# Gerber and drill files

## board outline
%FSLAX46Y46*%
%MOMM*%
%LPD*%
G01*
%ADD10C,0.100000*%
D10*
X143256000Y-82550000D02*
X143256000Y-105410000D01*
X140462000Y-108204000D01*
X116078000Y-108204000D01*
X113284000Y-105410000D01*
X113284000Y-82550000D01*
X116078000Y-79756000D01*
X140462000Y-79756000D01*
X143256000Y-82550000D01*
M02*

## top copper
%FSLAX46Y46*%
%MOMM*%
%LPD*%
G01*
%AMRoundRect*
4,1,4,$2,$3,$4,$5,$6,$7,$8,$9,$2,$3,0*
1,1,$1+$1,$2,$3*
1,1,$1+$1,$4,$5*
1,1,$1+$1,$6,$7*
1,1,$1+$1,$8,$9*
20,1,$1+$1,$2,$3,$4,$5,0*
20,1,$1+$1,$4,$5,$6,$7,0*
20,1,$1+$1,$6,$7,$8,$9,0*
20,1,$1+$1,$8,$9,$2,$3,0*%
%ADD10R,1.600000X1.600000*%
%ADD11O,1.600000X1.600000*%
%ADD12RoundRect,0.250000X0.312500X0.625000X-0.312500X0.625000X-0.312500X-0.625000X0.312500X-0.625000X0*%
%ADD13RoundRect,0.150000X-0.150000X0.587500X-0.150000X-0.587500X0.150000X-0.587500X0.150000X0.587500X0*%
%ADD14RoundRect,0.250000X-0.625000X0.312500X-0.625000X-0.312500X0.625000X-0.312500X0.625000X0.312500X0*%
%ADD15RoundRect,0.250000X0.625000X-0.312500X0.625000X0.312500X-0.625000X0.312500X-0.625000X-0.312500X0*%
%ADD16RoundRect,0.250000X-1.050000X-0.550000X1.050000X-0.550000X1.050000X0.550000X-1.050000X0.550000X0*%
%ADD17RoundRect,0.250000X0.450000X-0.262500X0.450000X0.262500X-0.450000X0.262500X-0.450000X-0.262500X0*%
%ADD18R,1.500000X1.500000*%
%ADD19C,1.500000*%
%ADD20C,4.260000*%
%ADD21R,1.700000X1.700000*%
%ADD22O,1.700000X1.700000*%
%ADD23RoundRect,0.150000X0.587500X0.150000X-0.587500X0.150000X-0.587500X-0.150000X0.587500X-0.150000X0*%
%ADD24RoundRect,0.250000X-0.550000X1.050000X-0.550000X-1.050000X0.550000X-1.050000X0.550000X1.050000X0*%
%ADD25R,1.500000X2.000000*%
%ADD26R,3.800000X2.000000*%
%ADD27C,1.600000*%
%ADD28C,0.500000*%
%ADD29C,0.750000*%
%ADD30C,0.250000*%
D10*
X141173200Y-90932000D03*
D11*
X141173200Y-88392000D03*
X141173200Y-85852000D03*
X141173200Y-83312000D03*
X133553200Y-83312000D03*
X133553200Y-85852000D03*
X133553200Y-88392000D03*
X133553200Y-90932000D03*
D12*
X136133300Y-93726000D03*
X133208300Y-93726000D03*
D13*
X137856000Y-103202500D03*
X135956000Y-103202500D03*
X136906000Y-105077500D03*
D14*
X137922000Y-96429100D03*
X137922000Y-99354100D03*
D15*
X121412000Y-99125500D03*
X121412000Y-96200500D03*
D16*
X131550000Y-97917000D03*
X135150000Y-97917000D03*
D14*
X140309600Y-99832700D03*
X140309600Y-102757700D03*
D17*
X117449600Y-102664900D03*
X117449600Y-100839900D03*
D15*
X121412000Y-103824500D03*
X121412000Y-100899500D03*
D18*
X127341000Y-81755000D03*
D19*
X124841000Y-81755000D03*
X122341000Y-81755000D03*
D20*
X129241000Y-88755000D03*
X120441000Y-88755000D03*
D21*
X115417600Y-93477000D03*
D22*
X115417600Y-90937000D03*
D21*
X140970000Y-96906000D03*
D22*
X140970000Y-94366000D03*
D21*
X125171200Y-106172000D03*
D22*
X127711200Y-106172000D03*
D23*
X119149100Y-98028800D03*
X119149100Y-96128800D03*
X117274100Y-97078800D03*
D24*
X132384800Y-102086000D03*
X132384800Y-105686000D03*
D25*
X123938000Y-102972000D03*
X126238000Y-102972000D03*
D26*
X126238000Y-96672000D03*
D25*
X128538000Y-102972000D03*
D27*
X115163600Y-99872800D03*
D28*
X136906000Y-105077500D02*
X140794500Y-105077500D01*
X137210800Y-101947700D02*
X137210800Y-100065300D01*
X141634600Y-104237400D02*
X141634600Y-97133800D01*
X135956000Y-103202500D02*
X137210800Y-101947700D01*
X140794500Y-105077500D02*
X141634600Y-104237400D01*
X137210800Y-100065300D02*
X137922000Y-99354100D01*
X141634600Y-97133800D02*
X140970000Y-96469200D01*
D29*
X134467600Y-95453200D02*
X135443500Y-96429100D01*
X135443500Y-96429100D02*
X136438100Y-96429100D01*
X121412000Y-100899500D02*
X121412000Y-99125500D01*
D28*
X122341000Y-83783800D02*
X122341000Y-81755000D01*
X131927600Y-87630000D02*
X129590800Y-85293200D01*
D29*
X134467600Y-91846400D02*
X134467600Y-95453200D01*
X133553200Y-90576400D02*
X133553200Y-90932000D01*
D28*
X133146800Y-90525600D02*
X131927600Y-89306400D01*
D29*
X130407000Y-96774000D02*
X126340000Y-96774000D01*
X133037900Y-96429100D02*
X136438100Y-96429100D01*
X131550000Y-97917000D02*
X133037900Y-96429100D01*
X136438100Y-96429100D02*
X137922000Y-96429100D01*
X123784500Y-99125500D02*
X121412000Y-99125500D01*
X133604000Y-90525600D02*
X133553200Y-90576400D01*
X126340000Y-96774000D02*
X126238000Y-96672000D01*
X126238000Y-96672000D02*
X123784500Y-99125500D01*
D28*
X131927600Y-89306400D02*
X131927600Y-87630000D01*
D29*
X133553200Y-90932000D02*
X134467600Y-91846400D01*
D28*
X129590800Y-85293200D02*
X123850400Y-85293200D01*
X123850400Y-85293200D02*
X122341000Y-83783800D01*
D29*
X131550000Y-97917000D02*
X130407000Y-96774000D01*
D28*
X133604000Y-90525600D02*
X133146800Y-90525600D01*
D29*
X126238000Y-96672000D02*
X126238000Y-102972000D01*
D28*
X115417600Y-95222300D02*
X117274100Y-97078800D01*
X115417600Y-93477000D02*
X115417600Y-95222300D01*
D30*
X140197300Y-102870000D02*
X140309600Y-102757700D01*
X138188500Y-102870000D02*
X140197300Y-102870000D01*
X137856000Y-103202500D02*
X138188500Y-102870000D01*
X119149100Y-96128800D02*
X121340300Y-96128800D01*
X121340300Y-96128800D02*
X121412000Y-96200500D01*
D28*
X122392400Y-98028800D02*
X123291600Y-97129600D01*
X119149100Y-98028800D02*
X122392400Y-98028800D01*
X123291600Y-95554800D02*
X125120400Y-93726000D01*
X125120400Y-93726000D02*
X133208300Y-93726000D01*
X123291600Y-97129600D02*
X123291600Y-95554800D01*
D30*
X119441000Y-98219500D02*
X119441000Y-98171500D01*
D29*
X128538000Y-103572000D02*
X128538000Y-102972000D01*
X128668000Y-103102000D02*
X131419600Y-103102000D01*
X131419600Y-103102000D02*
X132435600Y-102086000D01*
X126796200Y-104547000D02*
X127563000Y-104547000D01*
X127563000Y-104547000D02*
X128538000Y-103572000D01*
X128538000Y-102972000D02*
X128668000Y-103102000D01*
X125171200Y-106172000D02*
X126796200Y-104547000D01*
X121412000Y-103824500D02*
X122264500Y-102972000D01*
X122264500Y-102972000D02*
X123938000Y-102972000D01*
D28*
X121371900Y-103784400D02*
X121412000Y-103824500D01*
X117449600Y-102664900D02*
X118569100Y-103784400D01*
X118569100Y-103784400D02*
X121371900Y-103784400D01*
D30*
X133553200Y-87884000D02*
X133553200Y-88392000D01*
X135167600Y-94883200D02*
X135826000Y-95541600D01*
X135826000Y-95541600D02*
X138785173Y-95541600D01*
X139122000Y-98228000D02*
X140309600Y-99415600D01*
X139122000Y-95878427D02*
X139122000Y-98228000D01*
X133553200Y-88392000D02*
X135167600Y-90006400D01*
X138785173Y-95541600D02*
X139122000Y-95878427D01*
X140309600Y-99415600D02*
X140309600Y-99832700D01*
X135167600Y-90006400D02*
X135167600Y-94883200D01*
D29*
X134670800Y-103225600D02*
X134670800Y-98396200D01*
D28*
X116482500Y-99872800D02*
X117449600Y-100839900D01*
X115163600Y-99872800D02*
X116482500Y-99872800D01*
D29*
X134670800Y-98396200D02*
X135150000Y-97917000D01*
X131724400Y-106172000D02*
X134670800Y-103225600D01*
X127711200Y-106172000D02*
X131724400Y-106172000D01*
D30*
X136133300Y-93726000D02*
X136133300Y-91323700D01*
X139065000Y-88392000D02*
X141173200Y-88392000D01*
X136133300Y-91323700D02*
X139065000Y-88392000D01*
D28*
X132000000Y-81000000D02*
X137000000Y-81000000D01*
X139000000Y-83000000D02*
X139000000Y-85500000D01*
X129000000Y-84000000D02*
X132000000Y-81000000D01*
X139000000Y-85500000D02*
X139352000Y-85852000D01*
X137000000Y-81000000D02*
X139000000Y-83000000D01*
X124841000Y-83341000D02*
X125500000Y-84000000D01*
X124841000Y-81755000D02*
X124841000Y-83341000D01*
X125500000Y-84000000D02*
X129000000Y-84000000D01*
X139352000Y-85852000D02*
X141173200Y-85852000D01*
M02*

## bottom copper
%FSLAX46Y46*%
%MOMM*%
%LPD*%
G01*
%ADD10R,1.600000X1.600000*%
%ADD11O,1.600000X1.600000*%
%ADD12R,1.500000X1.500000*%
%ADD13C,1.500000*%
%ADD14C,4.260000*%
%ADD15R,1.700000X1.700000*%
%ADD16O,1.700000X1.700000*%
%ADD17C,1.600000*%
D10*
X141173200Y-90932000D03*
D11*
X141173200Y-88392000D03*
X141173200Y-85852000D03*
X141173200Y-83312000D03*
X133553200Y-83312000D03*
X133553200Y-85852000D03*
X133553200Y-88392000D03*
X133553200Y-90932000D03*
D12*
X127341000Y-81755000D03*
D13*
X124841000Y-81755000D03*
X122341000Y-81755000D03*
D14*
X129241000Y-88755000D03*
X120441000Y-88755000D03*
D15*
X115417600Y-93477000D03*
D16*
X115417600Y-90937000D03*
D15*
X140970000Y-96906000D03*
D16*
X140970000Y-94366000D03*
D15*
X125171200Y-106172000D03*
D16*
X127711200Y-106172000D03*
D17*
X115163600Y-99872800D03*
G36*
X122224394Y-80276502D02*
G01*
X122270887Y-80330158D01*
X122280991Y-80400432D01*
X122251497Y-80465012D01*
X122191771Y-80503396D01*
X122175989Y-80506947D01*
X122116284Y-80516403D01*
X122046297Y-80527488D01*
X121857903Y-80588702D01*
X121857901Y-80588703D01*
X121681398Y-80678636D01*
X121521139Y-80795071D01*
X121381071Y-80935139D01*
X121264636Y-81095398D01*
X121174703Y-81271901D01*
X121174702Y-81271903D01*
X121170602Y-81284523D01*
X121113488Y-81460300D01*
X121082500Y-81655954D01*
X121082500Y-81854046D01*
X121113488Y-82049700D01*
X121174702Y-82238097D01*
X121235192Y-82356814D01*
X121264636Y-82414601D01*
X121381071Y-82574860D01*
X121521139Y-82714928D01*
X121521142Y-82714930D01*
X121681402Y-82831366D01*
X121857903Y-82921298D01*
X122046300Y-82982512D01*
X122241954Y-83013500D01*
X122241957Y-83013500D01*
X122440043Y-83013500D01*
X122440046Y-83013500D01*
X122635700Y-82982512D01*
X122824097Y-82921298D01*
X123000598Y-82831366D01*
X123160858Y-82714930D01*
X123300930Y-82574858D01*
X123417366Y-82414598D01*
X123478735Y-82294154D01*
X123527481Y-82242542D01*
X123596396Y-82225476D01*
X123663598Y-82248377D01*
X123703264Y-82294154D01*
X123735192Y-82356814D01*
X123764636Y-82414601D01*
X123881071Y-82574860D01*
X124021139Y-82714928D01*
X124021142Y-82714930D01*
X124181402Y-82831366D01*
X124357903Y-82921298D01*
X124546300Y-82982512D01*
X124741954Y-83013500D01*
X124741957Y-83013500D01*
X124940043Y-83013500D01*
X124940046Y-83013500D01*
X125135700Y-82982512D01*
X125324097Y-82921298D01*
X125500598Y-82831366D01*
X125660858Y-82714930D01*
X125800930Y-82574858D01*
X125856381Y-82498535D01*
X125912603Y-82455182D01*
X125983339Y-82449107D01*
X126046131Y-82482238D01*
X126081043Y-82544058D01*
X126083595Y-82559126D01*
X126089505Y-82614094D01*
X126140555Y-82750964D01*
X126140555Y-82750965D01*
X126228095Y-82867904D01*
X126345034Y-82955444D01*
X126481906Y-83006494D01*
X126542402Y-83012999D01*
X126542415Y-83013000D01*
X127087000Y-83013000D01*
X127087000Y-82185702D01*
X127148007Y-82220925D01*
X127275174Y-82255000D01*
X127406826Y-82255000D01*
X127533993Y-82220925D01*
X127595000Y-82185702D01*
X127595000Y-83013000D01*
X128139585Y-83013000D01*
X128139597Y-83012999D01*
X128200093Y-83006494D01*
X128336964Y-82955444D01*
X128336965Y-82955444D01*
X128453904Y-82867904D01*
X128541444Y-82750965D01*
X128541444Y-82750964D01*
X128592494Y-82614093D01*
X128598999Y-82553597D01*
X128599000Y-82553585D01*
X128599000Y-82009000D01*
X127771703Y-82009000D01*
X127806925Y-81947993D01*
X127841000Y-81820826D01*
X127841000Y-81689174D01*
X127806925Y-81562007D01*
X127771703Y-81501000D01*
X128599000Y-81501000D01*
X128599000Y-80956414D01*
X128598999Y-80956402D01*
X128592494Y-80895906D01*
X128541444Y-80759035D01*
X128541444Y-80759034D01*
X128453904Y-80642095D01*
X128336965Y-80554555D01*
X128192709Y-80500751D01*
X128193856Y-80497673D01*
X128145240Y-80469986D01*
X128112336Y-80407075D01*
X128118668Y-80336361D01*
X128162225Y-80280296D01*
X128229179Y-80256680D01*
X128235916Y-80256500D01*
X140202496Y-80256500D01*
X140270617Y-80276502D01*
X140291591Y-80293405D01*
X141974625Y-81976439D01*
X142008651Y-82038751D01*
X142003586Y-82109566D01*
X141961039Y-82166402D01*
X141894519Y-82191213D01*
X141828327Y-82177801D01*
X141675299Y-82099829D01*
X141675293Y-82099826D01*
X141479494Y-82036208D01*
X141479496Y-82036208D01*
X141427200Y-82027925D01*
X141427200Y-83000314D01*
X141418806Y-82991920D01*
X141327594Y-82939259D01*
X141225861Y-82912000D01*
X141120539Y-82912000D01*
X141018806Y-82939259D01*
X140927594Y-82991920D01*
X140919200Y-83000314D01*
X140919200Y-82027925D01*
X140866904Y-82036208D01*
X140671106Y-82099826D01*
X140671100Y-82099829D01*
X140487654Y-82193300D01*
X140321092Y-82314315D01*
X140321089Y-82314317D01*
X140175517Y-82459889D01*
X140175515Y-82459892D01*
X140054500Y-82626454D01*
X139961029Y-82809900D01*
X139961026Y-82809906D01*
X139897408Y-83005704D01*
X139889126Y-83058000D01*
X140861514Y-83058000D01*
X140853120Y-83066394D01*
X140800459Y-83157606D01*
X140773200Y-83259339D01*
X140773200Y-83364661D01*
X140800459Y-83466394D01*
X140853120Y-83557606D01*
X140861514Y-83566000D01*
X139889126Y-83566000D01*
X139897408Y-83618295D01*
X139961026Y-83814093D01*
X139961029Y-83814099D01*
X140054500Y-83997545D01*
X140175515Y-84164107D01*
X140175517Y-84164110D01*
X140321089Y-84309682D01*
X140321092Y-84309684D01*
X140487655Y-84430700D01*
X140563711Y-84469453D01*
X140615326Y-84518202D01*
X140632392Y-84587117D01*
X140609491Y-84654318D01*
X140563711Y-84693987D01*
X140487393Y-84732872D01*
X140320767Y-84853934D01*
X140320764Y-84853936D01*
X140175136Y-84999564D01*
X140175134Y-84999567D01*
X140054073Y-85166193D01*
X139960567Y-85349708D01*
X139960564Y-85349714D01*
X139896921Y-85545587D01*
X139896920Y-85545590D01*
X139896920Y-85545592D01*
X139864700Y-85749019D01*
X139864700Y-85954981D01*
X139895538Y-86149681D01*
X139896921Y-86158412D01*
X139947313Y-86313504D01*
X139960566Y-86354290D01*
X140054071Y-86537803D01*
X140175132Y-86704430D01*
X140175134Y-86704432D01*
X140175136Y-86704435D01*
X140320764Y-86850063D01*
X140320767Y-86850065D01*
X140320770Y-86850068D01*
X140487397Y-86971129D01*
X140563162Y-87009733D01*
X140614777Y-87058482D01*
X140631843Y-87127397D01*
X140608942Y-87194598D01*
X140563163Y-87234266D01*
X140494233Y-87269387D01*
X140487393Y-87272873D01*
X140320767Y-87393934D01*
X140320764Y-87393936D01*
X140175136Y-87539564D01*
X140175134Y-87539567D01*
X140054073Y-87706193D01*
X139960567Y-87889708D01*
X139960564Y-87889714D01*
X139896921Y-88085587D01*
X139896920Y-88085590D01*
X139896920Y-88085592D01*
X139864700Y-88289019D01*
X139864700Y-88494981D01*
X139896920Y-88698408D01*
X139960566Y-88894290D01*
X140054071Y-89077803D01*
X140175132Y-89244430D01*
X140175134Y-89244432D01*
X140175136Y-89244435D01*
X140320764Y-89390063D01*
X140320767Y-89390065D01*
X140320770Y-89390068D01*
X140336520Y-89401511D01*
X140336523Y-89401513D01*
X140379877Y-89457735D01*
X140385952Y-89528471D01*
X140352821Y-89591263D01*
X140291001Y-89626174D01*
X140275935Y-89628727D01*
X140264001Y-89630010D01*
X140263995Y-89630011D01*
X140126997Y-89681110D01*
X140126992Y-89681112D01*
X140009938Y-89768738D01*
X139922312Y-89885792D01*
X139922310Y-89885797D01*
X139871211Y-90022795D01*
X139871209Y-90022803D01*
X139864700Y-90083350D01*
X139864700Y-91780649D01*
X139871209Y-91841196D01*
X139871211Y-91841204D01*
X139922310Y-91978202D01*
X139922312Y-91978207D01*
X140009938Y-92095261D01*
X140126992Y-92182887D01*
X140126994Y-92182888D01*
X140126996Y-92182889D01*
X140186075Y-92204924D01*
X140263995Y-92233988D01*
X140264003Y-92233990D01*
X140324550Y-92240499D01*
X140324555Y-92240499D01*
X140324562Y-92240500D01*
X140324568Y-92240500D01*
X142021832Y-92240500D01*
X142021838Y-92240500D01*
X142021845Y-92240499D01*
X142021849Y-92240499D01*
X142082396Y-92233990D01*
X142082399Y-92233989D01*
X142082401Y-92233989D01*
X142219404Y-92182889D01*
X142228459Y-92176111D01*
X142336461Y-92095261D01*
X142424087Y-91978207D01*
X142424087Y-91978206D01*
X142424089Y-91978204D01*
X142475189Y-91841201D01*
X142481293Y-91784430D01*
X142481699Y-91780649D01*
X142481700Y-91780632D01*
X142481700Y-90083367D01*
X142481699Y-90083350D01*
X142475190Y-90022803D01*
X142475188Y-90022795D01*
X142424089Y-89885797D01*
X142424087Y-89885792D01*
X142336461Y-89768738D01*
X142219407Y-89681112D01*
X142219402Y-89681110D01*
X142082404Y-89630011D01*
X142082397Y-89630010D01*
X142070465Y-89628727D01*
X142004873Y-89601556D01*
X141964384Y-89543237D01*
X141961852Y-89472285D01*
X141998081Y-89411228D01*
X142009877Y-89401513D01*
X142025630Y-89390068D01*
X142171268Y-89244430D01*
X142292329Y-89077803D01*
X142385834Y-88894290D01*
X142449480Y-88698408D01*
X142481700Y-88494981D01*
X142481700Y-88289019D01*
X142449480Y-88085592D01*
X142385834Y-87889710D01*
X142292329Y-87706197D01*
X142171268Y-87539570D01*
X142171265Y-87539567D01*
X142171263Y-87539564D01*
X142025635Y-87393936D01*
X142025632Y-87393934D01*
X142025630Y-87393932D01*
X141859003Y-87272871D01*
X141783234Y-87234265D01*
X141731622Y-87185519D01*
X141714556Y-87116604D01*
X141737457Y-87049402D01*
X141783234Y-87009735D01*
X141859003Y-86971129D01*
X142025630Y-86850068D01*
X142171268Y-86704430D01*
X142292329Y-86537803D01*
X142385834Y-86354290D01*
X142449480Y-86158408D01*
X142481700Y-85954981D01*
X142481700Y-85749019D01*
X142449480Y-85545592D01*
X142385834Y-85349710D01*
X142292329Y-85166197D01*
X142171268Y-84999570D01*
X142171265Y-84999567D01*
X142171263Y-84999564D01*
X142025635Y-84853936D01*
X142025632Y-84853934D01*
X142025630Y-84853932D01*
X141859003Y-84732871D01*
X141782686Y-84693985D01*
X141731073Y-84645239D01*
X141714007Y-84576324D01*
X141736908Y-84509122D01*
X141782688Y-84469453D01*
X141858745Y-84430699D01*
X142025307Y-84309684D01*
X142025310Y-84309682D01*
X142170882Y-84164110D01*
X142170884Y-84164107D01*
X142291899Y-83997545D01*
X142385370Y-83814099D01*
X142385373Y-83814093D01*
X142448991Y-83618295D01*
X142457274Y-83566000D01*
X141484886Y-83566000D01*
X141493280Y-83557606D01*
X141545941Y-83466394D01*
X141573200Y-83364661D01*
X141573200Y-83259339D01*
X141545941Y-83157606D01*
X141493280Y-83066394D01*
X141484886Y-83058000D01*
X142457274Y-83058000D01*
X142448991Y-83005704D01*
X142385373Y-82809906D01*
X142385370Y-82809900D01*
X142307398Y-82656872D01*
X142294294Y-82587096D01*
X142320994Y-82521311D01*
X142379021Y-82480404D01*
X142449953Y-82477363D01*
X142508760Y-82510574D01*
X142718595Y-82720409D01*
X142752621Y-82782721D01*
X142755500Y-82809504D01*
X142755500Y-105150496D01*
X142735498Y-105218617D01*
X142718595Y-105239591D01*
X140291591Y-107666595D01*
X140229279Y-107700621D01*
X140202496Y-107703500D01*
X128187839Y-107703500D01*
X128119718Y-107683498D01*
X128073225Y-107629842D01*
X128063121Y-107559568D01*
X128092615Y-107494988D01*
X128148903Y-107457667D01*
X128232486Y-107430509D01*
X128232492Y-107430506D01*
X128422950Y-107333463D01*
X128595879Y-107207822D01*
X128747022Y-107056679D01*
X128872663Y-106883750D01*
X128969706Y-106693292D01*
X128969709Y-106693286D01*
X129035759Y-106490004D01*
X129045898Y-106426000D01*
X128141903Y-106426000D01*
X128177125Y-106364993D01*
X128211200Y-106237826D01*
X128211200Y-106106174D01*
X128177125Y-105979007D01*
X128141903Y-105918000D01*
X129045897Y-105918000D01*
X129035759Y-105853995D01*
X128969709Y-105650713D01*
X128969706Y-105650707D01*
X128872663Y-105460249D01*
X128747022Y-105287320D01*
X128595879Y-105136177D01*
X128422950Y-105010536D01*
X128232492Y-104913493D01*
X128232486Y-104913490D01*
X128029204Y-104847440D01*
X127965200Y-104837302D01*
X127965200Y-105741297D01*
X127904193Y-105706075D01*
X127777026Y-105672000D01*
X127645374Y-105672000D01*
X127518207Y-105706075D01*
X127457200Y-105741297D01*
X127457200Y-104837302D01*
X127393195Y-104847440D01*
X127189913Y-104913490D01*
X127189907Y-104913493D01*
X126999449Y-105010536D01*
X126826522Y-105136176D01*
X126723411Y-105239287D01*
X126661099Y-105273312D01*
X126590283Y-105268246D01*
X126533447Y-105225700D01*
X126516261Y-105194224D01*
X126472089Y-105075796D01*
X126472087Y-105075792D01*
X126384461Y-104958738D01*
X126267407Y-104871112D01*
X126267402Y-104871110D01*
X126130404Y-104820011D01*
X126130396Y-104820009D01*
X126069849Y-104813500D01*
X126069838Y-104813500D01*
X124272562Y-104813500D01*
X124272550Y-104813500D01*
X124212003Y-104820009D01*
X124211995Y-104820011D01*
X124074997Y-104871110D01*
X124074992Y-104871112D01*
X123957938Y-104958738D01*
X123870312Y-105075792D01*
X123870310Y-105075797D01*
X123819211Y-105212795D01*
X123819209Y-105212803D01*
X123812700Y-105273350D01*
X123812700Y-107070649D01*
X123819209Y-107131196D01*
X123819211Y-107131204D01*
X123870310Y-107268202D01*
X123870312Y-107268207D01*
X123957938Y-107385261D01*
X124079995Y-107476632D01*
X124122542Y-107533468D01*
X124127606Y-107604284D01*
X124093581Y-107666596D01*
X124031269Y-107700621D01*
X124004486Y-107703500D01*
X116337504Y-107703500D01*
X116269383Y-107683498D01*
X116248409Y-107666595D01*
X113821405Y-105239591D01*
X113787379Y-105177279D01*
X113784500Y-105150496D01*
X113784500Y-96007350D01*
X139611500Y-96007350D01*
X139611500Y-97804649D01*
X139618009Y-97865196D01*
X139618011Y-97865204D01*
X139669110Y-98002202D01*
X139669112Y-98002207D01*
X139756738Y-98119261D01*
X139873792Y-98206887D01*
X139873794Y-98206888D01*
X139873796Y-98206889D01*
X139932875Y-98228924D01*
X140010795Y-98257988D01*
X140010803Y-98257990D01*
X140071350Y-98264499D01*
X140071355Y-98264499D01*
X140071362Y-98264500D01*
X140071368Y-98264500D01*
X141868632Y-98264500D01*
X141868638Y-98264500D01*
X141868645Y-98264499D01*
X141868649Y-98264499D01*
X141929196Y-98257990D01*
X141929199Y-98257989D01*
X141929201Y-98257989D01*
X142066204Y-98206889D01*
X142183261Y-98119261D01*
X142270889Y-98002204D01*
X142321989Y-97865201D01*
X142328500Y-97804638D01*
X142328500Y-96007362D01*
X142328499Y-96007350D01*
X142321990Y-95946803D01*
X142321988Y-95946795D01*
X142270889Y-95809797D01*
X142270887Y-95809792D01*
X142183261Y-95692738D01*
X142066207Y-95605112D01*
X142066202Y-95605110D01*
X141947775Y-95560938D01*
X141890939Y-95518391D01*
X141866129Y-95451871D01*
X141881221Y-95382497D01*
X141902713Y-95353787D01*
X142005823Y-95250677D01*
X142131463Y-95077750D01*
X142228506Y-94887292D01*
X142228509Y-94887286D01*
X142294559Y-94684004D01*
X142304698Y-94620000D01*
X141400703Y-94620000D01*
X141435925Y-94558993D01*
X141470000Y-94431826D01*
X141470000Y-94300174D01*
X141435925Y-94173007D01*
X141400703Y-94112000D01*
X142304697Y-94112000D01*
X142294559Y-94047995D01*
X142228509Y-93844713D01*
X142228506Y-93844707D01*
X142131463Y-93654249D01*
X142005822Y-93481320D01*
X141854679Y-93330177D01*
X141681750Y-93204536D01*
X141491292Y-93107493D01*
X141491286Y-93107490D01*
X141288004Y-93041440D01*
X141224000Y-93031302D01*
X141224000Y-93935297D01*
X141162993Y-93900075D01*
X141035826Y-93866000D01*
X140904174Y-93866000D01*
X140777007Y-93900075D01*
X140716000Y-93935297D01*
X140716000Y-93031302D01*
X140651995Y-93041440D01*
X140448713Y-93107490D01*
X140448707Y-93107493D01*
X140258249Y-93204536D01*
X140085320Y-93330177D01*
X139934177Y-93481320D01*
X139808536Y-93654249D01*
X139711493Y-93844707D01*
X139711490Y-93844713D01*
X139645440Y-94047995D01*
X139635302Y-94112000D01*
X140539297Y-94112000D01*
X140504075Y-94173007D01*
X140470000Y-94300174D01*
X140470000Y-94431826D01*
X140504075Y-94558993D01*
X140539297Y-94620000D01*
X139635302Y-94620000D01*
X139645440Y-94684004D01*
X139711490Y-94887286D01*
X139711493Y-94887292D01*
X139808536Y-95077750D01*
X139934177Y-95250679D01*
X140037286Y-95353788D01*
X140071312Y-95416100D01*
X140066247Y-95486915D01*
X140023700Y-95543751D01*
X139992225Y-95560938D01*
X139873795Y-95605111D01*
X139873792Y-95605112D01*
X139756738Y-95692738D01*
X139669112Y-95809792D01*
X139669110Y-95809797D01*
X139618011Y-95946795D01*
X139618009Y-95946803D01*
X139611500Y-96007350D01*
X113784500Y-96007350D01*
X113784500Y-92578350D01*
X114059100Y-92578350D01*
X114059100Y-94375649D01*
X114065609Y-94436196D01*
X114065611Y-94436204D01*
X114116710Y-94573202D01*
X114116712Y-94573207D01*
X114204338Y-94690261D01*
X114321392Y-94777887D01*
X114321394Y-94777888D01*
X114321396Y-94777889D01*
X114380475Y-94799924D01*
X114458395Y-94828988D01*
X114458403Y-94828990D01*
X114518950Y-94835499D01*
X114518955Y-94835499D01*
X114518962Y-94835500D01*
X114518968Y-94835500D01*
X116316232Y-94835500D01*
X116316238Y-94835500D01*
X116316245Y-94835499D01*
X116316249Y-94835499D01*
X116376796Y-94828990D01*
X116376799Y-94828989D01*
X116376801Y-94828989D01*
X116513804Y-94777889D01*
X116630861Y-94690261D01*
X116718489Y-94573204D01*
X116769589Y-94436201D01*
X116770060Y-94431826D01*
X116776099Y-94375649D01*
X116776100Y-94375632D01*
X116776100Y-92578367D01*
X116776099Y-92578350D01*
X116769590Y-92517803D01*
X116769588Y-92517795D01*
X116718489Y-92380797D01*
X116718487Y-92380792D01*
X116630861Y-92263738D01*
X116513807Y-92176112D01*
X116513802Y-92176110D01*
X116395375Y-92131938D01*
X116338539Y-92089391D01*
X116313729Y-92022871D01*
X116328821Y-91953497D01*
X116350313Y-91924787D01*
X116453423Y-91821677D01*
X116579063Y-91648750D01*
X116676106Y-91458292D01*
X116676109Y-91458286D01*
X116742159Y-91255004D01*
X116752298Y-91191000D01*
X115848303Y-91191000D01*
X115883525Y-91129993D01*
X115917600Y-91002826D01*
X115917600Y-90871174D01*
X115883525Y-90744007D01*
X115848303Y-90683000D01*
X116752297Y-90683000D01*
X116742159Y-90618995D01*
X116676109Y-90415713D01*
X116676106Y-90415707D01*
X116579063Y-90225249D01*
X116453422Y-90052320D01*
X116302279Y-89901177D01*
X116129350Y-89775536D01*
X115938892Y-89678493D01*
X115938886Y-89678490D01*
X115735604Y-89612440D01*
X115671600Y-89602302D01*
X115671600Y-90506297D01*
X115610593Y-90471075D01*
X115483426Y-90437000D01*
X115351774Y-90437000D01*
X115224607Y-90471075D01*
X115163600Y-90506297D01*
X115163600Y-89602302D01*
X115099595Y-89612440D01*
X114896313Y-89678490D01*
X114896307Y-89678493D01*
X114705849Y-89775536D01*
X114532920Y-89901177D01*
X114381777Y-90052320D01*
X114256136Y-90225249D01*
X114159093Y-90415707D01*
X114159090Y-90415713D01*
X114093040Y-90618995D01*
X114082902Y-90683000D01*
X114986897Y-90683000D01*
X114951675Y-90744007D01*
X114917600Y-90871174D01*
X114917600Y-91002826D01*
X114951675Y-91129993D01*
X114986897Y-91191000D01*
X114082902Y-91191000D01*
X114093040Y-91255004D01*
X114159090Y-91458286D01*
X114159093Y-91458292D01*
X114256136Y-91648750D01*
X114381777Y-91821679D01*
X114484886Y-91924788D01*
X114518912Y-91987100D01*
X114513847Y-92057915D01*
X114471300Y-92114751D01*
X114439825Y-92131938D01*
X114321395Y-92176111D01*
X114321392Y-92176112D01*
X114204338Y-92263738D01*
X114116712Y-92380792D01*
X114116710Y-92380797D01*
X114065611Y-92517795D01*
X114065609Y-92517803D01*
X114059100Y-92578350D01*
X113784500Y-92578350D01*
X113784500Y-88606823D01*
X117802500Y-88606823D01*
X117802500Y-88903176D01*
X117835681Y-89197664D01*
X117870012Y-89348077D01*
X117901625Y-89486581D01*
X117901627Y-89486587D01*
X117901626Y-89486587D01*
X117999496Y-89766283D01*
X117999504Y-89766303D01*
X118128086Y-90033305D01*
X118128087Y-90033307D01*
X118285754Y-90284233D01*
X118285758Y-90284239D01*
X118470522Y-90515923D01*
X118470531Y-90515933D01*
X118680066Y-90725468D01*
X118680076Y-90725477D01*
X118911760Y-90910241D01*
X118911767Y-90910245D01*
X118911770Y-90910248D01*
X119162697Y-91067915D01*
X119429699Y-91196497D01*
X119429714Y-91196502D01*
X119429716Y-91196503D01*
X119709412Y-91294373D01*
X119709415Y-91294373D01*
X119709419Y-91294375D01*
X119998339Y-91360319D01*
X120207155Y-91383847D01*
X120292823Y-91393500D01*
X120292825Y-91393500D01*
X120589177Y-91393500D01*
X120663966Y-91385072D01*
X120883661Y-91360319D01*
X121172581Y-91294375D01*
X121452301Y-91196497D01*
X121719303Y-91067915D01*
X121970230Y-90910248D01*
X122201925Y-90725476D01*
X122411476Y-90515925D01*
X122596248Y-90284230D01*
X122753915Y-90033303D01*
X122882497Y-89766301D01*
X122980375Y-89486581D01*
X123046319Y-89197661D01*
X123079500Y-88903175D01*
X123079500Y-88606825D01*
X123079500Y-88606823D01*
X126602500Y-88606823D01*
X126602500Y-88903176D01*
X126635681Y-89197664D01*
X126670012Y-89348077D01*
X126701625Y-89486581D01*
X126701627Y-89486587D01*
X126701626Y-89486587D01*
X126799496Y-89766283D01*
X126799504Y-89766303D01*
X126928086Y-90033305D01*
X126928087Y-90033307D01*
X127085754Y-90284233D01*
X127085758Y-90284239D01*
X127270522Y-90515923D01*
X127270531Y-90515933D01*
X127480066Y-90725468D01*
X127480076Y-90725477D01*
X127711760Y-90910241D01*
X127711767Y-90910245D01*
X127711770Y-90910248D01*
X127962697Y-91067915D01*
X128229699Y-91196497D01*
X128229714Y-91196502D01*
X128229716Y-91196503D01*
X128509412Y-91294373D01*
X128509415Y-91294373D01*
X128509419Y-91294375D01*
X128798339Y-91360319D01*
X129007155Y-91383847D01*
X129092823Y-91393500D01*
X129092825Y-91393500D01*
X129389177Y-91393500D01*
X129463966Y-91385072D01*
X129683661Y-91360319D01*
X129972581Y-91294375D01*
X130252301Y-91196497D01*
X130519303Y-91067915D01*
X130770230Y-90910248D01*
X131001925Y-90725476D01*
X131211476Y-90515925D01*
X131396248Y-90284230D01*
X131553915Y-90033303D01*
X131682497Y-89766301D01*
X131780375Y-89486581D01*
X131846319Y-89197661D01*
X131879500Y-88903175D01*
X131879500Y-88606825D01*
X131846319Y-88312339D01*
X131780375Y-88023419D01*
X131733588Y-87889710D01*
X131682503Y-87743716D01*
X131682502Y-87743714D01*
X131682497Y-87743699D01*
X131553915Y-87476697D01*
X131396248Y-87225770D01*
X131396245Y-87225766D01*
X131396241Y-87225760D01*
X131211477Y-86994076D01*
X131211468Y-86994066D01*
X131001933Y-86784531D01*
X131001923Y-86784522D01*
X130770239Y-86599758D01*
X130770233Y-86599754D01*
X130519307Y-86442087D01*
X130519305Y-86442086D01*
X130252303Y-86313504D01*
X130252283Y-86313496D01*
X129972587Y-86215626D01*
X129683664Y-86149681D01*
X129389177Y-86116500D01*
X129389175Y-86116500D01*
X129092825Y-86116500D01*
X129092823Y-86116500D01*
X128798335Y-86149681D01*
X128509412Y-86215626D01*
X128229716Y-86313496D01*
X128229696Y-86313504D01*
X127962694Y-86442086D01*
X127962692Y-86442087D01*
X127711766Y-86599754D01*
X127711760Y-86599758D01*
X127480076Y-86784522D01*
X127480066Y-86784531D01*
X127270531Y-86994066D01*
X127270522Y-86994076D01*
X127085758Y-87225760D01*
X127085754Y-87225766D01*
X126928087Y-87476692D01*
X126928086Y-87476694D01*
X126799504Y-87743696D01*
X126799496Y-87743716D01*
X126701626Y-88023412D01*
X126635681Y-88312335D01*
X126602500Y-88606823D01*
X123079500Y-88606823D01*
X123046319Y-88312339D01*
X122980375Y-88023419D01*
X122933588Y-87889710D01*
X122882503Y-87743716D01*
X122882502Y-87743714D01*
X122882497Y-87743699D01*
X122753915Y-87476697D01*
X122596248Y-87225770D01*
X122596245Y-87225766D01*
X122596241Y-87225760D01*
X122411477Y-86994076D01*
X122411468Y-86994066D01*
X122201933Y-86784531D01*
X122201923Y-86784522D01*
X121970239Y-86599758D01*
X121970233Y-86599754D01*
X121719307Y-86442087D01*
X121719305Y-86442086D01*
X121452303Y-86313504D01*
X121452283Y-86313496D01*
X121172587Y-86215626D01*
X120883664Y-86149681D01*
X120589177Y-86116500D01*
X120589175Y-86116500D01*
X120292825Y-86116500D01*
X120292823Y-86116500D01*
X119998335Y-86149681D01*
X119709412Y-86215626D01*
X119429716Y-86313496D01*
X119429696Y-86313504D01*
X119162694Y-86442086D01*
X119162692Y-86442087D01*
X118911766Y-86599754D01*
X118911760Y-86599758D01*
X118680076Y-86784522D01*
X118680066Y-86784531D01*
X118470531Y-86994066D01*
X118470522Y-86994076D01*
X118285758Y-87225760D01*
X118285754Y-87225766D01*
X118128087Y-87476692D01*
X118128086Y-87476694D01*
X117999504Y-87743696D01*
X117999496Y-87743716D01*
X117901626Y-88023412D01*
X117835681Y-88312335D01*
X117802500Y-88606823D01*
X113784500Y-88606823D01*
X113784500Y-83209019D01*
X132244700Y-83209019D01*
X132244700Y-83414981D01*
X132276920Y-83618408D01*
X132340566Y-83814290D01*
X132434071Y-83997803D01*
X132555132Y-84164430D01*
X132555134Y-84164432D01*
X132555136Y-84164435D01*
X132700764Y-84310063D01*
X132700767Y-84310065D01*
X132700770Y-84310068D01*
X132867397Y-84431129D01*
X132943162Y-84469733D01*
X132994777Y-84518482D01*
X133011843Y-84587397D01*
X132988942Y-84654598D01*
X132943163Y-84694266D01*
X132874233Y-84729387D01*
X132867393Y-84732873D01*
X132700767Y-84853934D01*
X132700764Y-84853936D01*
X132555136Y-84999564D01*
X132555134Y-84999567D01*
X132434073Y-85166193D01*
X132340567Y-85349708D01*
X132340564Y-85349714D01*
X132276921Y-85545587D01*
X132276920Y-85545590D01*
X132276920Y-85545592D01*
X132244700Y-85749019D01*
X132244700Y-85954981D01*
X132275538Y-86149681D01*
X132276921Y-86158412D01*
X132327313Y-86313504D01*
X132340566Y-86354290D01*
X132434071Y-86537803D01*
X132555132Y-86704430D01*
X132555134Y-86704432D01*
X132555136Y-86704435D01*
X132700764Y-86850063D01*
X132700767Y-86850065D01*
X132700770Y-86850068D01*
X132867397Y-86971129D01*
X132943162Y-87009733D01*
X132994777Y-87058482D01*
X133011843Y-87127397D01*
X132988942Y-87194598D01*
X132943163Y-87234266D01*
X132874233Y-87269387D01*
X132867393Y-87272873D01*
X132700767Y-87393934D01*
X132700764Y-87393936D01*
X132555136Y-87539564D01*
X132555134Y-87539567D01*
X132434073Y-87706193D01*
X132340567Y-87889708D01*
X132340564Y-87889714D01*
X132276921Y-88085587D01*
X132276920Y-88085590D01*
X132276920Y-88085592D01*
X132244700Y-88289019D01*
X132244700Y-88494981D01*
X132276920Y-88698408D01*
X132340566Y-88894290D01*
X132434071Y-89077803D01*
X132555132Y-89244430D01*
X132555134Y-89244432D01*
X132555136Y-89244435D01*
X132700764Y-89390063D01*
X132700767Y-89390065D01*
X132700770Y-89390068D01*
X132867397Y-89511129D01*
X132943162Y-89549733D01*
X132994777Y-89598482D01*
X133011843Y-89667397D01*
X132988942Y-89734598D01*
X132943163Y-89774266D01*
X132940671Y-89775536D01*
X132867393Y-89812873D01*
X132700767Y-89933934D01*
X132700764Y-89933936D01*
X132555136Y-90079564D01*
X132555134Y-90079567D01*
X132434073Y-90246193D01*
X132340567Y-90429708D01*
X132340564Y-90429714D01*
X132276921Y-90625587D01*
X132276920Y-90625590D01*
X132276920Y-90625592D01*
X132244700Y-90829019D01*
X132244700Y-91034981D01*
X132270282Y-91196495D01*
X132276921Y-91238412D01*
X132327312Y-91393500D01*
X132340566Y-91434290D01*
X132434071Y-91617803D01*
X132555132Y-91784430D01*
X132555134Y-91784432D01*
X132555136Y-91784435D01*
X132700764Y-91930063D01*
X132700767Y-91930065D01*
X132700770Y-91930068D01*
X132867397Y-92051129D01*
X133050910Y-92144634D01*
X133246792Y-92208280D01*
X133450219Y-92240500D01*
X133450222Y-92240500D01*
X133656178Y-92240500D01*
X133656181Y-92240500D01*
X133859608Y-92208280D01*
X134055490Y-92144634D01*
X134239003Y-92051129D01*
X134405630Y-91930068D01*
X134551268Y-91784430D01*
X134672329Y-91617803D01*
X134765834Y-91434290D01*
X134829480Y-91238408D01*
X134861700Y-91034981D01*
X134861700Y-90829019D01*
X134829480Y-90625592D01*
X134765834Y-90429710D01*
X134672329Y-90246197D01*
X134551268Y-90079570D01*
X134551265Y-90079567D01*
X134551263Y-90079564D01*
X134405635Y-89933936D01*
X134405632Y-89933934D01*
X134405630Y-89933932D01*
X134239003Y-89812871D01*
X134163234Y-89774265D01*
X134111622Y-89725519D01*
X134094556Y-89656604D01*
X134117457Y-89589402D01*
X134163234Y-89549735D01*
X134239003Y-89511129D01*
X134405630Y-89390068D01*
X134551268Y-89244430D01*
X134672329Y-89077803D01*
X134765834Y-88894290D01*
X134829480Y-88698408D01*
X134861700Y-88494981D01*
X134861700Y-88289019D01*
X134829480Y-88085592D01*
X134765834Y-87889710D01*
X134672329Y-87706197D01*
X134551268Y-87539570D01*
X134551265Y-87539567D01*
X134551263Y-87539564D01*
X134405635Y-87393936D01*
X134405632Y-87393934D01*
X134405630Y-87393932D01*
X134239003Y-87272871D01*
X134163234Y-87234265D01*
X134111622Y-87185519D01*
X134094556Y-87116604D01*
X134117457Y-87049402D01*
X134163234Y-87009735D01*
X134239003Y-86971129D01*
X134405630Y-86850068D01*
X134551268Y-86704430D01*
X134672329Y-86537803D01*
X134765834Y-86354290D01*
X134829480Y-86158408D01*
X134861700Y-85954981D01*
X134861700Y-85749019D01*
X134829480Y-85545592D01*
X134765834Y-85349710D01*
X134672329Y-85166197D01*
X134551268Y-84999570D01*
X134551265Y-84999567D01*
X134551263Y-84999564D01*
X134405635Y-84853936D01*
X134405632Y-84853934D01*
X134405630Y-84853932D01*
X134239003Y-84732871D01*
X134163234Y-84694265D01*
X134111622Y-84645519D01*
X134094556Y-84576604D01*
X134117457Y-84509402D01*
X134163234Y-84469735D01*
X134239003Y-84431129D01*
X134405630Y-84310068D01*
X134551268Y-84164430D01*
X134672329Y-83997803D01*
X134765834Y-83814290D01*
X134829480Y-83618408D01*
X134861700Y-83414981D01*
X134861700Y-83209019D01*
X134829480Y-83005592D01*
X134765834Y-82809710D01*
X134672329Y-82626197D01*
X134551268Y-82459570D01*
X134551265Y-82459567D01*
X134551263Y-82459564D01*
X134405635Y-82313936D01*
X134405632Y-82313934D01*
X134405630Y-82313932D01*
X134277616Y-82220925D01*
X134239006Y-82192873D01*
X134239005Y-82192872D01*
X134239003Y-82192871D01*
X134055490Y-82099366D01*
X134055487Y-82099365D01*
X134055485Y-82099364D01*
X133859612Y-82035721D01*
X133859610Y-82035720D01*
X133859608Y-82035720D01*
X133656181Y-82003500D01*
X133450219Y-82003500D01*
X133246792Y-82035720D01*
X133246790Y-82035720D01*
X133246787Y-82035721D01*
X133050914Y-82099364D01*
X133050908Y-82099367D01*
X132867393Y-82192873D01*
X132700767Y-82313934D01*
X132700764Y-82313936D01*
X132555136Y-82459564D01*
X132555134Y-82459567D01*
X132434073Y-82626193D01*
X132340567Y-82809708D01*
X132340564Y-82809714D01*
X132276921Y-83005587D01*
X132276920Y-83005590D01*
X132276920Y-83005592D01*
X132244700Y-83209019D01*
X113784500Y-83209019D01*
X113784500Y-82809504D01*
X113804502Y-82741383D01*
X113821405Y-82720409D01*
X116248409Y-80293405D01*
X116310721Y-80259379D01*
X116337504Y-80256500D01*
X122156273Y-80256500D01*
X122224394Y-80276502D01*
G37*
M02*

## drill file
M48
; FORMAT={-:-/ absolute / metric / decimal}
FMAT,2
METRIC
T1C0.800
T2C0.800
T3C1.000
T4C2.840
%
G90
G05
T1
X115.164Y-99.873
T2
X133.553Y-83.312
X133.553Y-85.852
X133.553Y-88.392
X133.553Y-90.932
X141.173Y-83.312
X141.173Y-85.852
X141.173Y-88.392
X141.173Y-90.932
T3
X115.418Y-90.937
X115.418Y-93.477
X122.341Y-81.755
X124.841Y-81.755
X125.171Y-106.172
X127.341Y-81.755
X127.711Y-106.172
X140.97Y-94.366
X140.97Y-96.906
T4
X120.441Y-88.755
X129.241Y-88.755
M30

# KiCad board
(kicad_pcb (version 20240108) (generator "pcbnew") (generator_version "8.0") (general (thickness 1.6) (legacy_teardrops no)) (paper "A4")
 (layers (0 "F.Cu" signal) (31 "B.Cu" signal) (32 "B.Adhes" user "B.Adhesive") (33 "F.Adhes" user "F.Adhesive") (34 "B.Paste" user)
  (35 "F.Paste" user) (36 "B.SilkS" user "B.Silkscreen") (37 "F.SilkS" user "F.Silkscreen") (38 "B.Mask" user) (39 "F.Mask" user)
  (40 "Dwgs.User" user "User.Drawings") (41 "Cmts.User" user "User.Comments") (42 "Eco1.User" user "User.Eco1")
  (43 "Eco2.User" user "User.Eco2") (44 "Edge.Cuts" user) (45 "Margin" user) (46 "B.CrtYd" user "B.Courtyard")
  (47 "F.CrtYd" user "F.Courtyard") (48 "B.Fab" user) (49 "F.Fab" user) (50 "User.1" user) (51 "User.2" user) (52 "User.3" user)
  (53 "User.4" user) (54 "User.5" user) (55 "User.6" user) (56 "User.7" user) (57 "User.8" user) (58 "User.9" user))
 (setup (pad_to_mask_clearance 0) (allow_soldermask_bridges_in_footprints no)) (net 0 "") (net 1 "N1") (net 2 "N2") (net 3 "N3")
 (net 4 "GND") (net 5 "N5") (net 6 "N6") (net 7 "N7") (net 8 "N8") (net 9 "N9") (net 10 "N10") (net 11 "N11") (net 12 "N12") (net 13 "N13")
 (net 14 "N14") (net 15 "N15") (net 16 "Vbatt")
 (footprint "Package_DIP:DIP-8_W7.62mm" (layer "F.Cu") (at 141.1732 90.932 180)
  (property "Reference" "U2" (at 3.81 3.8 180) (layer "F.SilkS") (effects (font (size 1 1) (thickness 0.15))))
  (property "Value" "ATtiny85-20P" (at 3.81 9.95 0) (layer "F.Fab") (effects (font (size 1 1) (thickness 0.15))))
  (pad "1" thru_hole rect (at 0 0 180) (size 1.6 1.6) (drill 0.8) (layers "*.Cu" "*.Mask") (remove_unused_layers no) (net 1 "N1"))
  (pad "2" thru_hole oval (at 0 2.54 180) (size 1.6 1.6) (drill 0.8) (layers "*.Cu" "*.Mask") (remove_unused_layers no) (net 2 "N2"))
  (pad "3" thru_hole oval (at 0 5.08 180) (size 1.6 1.6) (drill 0.8) (layers "*.Cu" "*.Mask") (remove_unused_layers no) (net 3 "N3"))
  (pad "4" thru_hole oval (at 0 7.62 180) (size 1.6 1.6) (drill 0.8) (layers "*.Cu" "*.Mask") (remove_unused_layers no) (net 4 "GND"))
  (pad "5" thru_hole oval (at 7.62 7.62 180) (size 1.6 1.6) (drill 0.8) (layers "*.Cu" "*.Mask") (remove_unused_layers no) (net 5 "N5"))
  (pad "6" thru_hole oval (at 7.62 5.08 180) (size 1.6 1.6) (drill 0.8) (layers "*.Cu" "*.Mask") (remove_unused_layers no) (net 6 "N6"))
  (pad "7" thru_hole oval (at 7.62 2.54 180) (size 1.6 1.6) (drill 0.8) (layers "*.Cu" "*.Mask") (remove_unused_layers no) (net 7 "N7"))
  (pad "8" thru_hole oval (at 7.62 0 180) (size 1.6 1.6) (drill 0.8) (layers "*.Cu" "*.Mask") (remove_unused_layers no) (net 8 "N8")))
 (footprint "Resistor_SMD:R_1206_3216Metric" (layer "F.Cu") (at 134.6708 93.726 180)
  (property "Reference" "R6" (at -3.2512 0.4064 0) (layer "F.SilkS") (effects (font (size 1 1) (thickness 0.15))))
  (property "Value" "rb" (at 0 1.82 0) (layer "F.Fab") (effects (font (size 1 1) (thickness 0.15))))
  (pad "1" smd roundrect (at -1.4625 0 180) (size 1.125 1.75) (layers "F.Cu" "F.Paste" "F.Mask") (roundrect_rratio 0.2222222222)
   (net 2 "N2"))
  (pad "2" smd roundrect (at 1.4625 0 180) (size 1.125 1.75) (layers "F.Cu" "F.Paste" "F.Mask") (roundrect_rratio 0.2222222222) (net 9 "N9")))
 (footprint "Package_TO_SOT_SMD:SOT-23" (layer "F.Cu") (at 136.906 104.14 -90)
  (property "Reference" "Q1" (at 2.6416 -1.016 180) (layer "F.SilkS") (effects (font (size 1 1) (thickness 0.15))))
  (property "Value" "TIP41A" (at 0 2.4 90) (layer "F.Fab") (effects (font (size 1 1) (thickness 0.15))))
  (pad "1" smd roundrect (at -0.9375 -0.95 270) (size 1.475 0.6) (layers "F.Cu" "F.Paste" "F.Mask") (roundrect_rratio 0.25) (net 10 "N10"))
  (pad "2" smd roundrect (at -0.9375 0.95 270) (size 1.475 0.6) (layers "F.Cu" "F.Paste" "F.Mask") (roundrect_rratio 0.25) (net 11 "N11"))
  (pad "3" smd roundrect (at 0.9375 0 270) (size 1.475 0.6) (layers "F.Cu" "F.Paste" "F.Mask") (roundrect_rratio 0.25) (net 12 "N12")))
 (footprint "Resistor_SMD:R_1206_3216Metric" (layer "F.Cu") (at 137.922 97.8916 -90)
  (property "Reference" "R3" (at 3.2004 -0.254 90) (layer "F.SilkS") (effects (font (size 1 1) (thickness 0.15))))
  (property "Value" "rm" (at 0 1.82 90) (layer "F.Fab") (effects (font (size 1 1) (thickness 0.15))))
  (pad "1" smd roundrect (at -1.4625 0 270) (size 1.125 1.75) (layers "F.Cu" "F.Paste" "F.Mask") (roundrect_rratio 0.2222222222)
   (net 8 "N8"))
  (pad "2" smd roundrect (at 1.4625 0 270) (size 1.125 1.75) (layers "F.Cu" "F.Paste" "F.Mask") (roundrect_rratio 0.2222222222)
   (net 12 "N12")))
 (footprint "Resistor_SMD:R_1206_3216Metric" (layer "F.Cu") (at 121.412 97.663 90)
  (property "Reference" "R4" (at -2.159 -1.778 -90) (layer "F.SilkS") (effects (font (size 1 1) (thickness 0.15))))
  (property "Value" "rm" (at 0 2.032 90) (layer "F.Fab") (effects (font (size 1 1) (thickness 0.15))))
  (pad "1" smd roundrect (at -1.4625 0 90) (size 1.125 1.75) (layers "F.Cu" "F.Paste" "F.Mask") (roundrect_rratio 0.2222222222) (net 8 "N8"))
  (pad "2" smd roundrect (at 1.4625 0 90) (size 1.125 1.75) (layers "F.Cu" "F.Paste" "F.Mask") (roundrect_rratio 0.2222222222)
   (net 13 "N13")))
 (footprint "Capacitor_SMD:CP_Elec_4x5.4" (layer "F.Cu") (at 133.35 97.917)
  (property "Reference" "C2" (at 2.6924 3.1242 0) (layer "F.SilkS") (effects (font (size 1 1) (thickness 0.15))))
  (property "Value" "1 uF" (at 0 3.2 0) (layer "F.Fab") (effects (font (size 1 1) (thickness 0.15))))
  (pad "1" smd roundrect (at -1.8 0) (size 2.6 1.6) (layers "F.Cu" "F.Paste" "F.Mask") (roundrect_rratio 0.15625) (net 8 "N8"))
  (pad "2" smd roundrect (at 1.8 0) (size 2.6 1.6) (layers "F.Cu" "F.Paste" "F.Mask") (roundrect_rratio 0.15625) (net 4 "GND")))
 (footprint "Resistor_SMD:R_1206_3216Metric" (layer "F.Cu") (at 140.3096 101.2952 -90)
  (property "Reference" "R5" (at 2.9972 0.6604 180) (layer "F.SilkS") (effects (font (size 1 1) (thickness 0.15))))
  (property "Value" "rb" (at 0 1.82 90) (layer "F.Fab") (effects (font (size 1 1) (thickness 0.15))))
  (pad "1" smd roundrect (at -1.4625 0 270) (size 1.125 1.75) (layers "F.Cu" "F.Paste" "F.Mask") (roundrect_rratio 0.2222222222)
   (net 7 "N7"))
  (pad "2" smd roundrect (at 1.4625 0 270) (size 1.125 1.75) (layers "F.Cu" "F.Paste" "F.Mask") (roundrect_rratio 0.2222222222)
   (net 10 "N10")))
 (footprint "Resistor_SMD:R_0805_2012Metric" (layer "F.Cu") (at 117.4496 101.7524 90)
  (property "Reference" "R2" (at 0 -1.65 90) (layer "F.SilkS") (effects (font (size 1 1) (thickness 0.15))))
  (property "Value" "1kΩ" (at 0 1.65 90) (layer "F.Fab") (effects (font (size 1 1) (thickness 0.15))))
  (pad "1" smd roundrect (at -0.9125 0 90) (size 1.025 1.4) (layers "F.Cu" "F.Paste" "F.Mask") (roundrect_rratio 0.243902) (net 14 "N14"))
  (pad "2" smd roundrect (at 0.9125 0 90) (size 1.025 1.4) (layers "F.Cu" "F.Paste" "F.Mask") (roundrect_rratio 0.243902) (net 4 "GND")))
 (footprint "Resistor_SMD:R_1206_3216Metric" (layer "F.Cu") (at 121.412 102.362 90)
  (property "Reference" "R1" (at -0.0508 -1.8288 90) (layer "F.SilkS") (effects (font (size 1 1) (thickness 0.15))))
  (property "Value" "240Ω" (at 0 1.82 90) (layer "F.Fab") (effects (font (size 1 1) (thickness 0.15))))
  (pad "1" smd roundrect (at -1.4625 0 90) (size 1.125 1.75) (layers "F.Cu" "F.Paste" "F.Mask") (roundrect_rratio 0.2222222222)
   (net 14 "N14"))
  (pad "2" smd roundrect (at 1.4625 0 90) (size 1.125 1.75) (layers "F.Cu" "F.Paste" "F.Mask") (roundrect_rratio 0.2222222222) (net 8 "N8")))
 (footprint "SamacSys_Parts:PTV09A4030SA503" (layer "F.Cu") (at 127.341 81.755 180)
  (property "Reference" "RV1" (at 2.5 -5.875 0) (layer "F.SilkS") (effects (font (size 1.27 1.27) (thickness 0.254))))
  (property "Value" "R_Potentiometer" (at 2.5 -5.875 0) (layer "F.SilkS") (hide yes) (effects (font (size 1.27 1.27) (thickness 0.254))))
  (pad "1" thru_hole rect (at 0 0 180) (size 1.5 1.5) (drill 1) (layers "*.Cu" "*.Mask") (remove_unused_layers no) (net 4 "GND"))
  (pad "2" thru_hole circle (at 2.5 0 180) (size 1.5 1.5) (drill 1) (layers "*.Cu" "*.Mask") (remove_unused_layers no) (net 3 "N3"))
  (pad "3" thru_hole circle (at 5 0 180) (size 1.5 1.5) (drill 1) (layers "*.Cu" "*.Mask") (remove_unused_layers no) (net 8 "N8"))
  (pad "MH1" thru_hole circle (at -1.9 -7 180) (size 4.26 4.26) (drill 2.84) (layers "*.Cu" "*.Mask") (remove_unused_layers no))
  (pad "MH2" thru_hole circle (at 6.9 -7 180) (size 4.26 4.26) (drill 2.84) (layers "*.Cu" "*.Mask") (remove_unused_layers no)))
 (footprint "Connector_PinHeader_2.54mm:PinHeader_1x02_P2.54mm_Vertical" (layer "F.Cu") (at 115.4176 93.477 180)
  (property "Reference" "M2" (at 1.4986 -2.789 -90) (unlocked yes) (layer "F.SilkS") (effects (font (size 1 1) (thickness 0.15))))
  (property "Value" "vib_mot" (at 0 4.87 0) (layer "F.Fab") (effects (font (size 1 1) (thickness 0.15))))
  (pad "1" thru_hole rect (at 0 0 180) (size 1.7 1.7) (drill 1) (layers "*.Cu" "*.Mask") (remove_unused_layers no) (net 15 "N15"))
  (pad "2" thru_hole oval (at 0 2.54 180) (size 1.7 1.7) (drill 1) (layers "*.Cu" "*.Mask") (remove_unused_layers no) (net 4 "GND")))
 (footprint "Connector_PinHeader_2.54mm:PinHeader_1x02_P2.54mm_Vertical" (layer "F.Cu") (at 140.97 96.906 180)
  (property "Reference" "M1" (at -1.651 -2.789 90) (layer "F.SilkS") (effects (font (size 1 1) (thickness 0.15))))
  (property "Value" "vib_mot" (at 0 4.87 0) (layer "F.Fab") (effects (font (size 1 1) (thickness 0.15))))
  (pad "1" thru_hole rect (at 0 0 180) (size 1.7 1.7) (drill 1) (layers "*.Cu" "*.Mask") (remove_unused_layers no) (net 11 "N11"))
  (pad "2" thru_hole oval (at 0 2.54 180) (size 1.7 1.7) (drill 1) (layers "*.Cu" "*.Mask") (remove_unused_layers no) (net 4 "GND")))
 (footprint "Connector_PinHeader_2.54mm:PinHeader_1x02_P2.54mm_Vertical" (layer "F.Cu") (at 125.1712 106.172 90)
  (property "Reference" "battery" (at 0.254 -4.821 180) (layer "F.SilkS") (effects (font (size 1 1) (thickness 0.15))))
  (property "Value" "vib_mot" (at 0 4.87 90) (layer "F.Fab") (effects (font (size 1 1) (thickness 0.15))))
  (pad "1" thru_hole rect (at 0 0 90) (size 1.7 1.7) (drill 1) (layers "*.Cu" "*.Mask") (remove_unused_layers no) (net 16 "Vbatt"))
  (pad "2" thru_hole oval (at 0 2.54 90) (size 1.7 1.7) (drill 1) (layers "*.Cu" "*.Mask") (remove_unused_layers no) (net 4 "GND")))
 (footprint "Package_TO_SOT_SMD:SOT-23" (layer "F.Cu") (at 118.2116 97.0788 180)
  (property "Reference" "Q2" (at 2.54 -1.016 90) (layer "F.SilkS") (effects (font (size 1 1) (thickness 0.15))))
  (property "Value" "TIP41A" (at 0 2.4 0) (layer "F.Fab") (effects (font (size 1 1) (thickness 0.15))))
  (pad "1" smd roundrect (at -0.9375 -0.95 180) (size 1.475 0.6) (layers "F.Cu" "F.Paste" "F.Mask") (roundrect_rratio 0.25) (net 9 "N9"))
  (pad "2" smd roundrect (at -0.9375 0.95 180) (size 1.475 0.6) (layers "F.Cu" "F.Paste" "F.Mask") (roundrect_rratio 0.25) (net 13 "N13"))
  (pad "3" smd roundrect (at 0.9375 0 180) (size 1.475 0.6) (layers "F.Cu" "F.Paste" "F.Mask") (roundrect_rratio 0.25) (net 15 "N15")))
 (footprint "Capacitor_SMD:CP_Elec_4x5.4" (layer "F.Cu") (at 132.3848 103.886 -90)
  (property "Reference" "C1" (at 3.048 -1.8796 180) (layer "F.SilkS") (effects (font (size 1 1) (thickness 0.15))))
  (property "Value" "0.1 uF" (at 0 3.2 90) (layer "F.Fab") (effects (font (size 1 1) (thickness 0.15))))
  (pad "1" smd roundrect (at -1.8 0 270) (size 2.6 1.6) (layers "F.Cu" "F.Paste" "F.Mask") (roundrect_rratio 0.15625) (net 16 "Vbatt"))
  (pad "2" smd roundrect (at 1.8 0 270) (size 2.6 1.6) (layers "F.Cu" "F.Paste" "F.Mask") (roundrect_rratio 0.15625) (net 4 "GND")))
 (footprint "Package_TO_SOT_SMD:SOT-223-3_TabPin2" (layer "F.Cu") (at 126.238 99.822 90)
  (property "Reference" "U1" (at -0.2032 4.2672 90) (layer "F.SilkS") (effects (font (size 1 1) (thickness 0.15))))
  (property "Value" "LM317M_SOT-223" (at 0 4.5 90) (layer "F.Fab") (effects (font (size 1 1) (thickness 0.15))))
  (pad "1" smd rect (at -3.15 -2.3 90) (size 2 1.5) (layers "F.Cu" "F.Paste" "F.Mask") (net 14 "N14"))
  (pad "2" smd rect (at -3.15 0 90) (size 2 1.5) (layers "F.Cu" "F.Paste" "F.Mask") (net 8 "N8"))
  (pad "2" smd rect (at 3.15 0 90) (size 2 3.8) (layers "F.Cu" "F.Paste" "F.Mask") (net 8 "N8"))
  (pad "3" smd rect (at -3.15 2.3 90) (size 2 1.5) (layers "F.Cu" "F.Paste" "F.Mask") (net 16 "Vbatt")))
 (gr_poly
  (pts (xy 143.256 82.55) (xy 143.256 105.41) (xy 140.462 108.204) (xy 116.078 108.204) (xy 113.284 105.41) (xy 113.284 82.55)
   (xy 116.078 79.756) (xy 140.462 79.756))
  (stroke (width 0.1) (type solid)) (fill none) (layer "Edge.Cuts"))
 (segment (start 136.906 105.0775) (end 140.7945 105.0775) (width 0.5) (layer "F.Cu") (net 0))
 (segment (start 137.2108 101.9477) (end 137.2108 100.0653) (width 0.5) (layer "F.Cu") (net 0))
 (segment (start 141.6346 104.2374) (end 141.6346 97.1338) (width 0.5) (layer "F.Cu") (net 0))
 (segment (start 135.956 103.2025) (end 137.2108 101.9477) (width 0.5) (layer "F.Cu") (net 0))
 (segment (start 140.7945 105.0775) (end 141.6346 104.2374) (width 0.5) (layer "F.Cu") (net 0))
 (segment (start 137.2108 100.0653) (end 137.922 99.3541) (width 0.5) (layer "F.Cu") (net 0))
 (segment (start 141.6346 97.1338) (end 140.97 96.4692) (width 0.5) (layer "F.Cu") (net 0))
 (segment (start 134.4676 95.4532) (end 135.4435 96.4291) (width 0.75) (layer "F.Cu") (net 8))
 (segment (start 135.4435 96.4291) (end 136.4381 96.4291) (width 0.75) (layer "F.Cu") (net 8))
 (segment (start 121.412 100.8995) (end 121.412 99.1255) (width 0.75) (layer "F.Cu") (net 8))
 (segment (start 122.341 83.7838) (end 122.341 81.755) (width 0.5) (layer "F.Cu") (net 8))
 (segment (start 131.9276 87.63) (end 129.5908 85.2932) (width 0.5) (layer "F.Cu") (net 8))
 (segment (start 134.4676 91.8464) (end 134.4676 95.4532) (width 0.75) (layer "F.Cu") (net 8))
 (segment (start 133.5532 90.5764) (end 133.5532 90.932) (width 0.75) (layer "F.Cu") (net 8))
 (segment (start 133.1468 90.5256) (end 131.9276 89.3064) (width 0.5) (layer "F.Cu") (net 8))
 (segment (start 130.407 96.774) (end 126.34 96.774) (width 0.75) (layer "F.Cu") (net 8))
 (segment (start 133.0379 96.4291) (end 136.4381 96.4291) (width 0.75) (layer "F.Cu") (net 8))
 (segment (start 131.55 97.917) (end 133.0379 96.4291) (width 0.75) (layer "F.Cu") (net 8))
 (segment (start 136.4381 96.4291) (end 137.922 96.4291) (width 0.75) (layer "F.Cu") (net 8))
 (segment (start 123.7845 99.1255) (end 121.412 99.1255) (width 0.75) (layer "F.Cu") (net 8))
 (segment (start 133.604 90.5256) (end 133.5532 90.5764) (width 0.75) (layer "F.Cu") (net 8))
 (segment (start 126.34 96.774) (end 126.238 96.672) (width 0.75) (layer "F.Cu") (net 8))
 (segment (start 126.238 96.672) (end 123.7845 99.1255) (width 0.75) (layer "F.Cu") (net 8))
 (segment (start 131.9276 89.3064) (end 131.9276 87.63) (width 0.5) (layer "F.Cu") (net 8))
 (segment (start 133.5532 90.932) (end 134.4676 91.8464) (width 0.75) (layer "F.Cu") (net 8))
 (segment (start 129.5908 85.2932) (end 123.8504 85.2932) (width 0.5) (layer "F.Cu") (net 8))
 (segment (start 123.8504 85.2932) (end 122.341 83.7838) (width 0.5) (layer "F.Cu") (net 8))
 (segment (start 131.55 97.917) (end 130.407 96.774) (width 0.75) (layer "F.Cu") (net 8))
 (segment (start 133.604 90.5256) (end 133.1468 90.5256) (width 0.5) (layer "F.Cu") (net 8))
 (segment (start 126.238 96.672) (end 126.238 102.972) (width 0.75) (layer "F.Cu") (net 8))
 (segment (start 115.4176 95.2223) (end 117.2741 97.0788) (width 0.5) (layer "F.Cu") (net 15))
 (segment (start 115.4176 93.477) (end 115.4176 95.2223) (width 0.5) (layer "F.Cu") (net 15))
 (segment (start 140.1973 102.87) (end 140.3096 102.7577) (width 0.25) (layer "F.Cu") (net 10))
 (segment (start 138.1885 102.87) (end 140.1973 102.87) (width 0.25) (layer "F.Cu") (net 10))
 (segment (start 137.856 103.2025) (end 138.1885 102.87) (width 0.25) (layer "F.Cu") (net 10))
 (segment (start 119.1491 96.1288) (end 121.3403 96.1288) (width 0.25) (layer "F.Cu") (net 13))
 (segment (start 121.3403 96.1288) (end 121.412 96.2005) (width 0.25) (layer "F.Cu") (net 13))
 (segment (start 122.3924 98.0288) (end 123.2916 97.1296) (width 0.5) (layer "F.Cu") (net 9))
 (segment (start 119.1491 98.0288) (end 122.3924 98.0288) (width 0.5) (layer "F.Cu") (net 9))
 (segment (start 123.2916 95.5548) (end 125.1204 93.726) (width 0.5) (layer "F.Cu") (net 9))
 (segment (start 125.1204 93.726) (end 133.2083 93.726) (width 0.5) (layer "F.Cu") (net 9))
 (segment (start 123.2916 97.1296) (end 123.2916 95.5548) (width 0.5) (layer "F.Cu") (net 9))
 (segment (start 119.441 98.2195) (end 119.441 98.1715) (width 0.25) (layer "F.Cu") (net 9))
 (segment (start 128.538 103.572) (end 128.538 102.972) (width 0.75) (layer "F.Cu") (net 16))
 (segment (start 128.668 103.102) (end 131.4196 103.102) (width 0.75) (layer "F.Cu") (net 16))
 (segment (start 131.4196 103.102) (end 132.4356 102.086) (width 0.75) (layer "F.Cu") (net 16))
 (segment (start 126.7962 104.547) (end 127.563 104.547) (width 0.75) (layer "F.Cu") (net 16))
 (segment (start 127.563 104.547) (end 128.538 103.572) (width 0.75) (layer "F.Cu") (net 16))
 (segment (start 128.538 102.972) (end 128.668 103.102) (width 0.75) (layer "F.Cu") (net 16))
 (segment (start 125.1712 106.172) (end 126.7962 104.547) (width 0.75) (layer "F.Cu") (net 16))
 (segment (start 121.412 103.8245) (end 122.2645 102.972) (width 0.75) (layer "F.Cu") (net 14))
 (segment (start 122.2645 102.972) (end 123.938 102.972) (width 0.75) (layer "F.Cu") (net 14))
 (segment (start 121.3719 103.7844) (end 121.412 103.8245) (width 0.5) (layer "F.Cu") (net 14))
 (segment (start 117.4496 102.6649) (end 118.5691 103.7844) (width 0.5) (layer "F.Cu") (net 14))
 (segment (start 118.5691 103.7844) (end 121.3719 103.7844) (width 0.5) (layer "F.Cu") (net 14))
 (segment (start 133.5532 87.884) (end 133.5532 88.392) (width 0.25) (layer "F.Cu") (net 7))
 (segment (start 135.1676 94.8832) (end 135.826 95.5416) (width 0.25) (layer "F.Cu") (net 7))
 (segment (start 135.826 95.5416) (end 138.785173 95.5416) (width 0.25) (layer "F.Cu") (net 7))
 (segment (start 139.122 98.228) (end 140.3096 99.4156) (width 0.25) (layer "F.Cu") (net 7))
 (segment (start 139.122 95.878427) (end 139.122 98.228) (width 0.25) (layer "F.Cu") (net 7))
 (segment (start 133.5532 88.392) (end 135.1676 90.0064) (width 0.25) (layer "F.Cu") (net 7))
 (segment (start 138.785173 95.5416) (end 139.122 95.878427) (width 0.25) (layer "F.Cu") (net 7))
 (segment (start 140.3096 99.4156) (end 140.3096 99.8327) (width 0.25) (layer "F.Cu") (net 7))
 (segment (start 135.1676 90.0064) (end 135.1676 94.8832) (width 0.25) (layer "F.Cu") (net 7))
 (segment (start 134.6708 103.2256) (end 134.6708 98.3962) (width 0.75) (layer "F.Cu") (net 4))
 (segment (start 116.4825 99.8728) (end 117.4496 100.8399) (width 0.5) (layer "F.Cu") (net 4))
 (segment (start 115.1636 99.8728) (end 116.4825 99.8728) (width 0.5) (layer "F.Cu") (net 4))
 (segment (start 134.6708 98.3962) (end 135.15 97.917) (width 0.75) (layer "F.Cu") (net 4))
 (segment (start 131.7244 106.172) (end 134.6708 103.2256) (width 0.75) (layer "F.Cu") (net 4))
 (segment (start 127.7112 106.172) (end 131.7244 106.172) (width 0.75) (layer "F.Cu") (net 4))
 (via (at 115.1636 99.8728) (size 1.6) (drill 0.8) (layers "F.Cu" "B.Cu") (free yes) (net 4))
 (segment (start 136.1333 93.726) (end 136.1333 91.3237) (width 0.25) (layer "F.Cu") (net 2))
 (segment (start 139.065 88.392) (end 141.1732 88.392) (width 0.25) (layer "F.Cu") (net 2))
 (segment (start 136.1333 91.3237) (end 139.065 88.392) (width 0.25) (layer "F.Cu") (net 2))
 (segment (start 132 81) (end 137 81) (width 0.5) (layer "F.Cu") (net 3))
 (segment (start 139 83) (end 139 85.5) (width 0.5) (layer "F.Cu") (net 3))
 (segment (start 129 84) (end 132 81) (width 0.5) (layer "F.Cu") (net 3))
 (segment (start 139 85.5) (end 139.352 85.852) (width 0.5) (layer "F.Cu") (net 3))
 (segment (start 137 81) (end 139 83) (width 0.5) (layer "F.Cu") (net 3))
 (segment (start 124.841 83.341) (end 125.5 84) (width 0.5) (layer "F.Cu") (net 3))
 (segment (start 124.841 81.755) (end 124.841 83.341) (width 0.5) (layer "F.Cu") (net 3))
 (segment (start 125.5 84) (end 129 84) (width 0.5) (layer "F.Cu") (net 3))
 (segment (start 139.352 85.852) (end 141.1732 85.852) (width 0.5) (layer "F.Cu") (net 3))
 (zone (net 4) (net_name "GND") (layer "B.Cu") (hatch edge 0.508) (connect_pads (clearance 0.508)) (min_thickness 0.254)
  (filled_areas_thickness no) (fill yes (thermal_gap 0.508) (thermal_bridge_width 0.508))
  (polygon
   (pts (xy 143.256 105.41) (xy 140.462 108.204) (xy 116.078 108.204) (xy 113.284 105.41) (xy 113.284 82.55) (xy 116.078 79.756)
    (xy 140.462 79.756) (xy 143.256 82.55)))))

